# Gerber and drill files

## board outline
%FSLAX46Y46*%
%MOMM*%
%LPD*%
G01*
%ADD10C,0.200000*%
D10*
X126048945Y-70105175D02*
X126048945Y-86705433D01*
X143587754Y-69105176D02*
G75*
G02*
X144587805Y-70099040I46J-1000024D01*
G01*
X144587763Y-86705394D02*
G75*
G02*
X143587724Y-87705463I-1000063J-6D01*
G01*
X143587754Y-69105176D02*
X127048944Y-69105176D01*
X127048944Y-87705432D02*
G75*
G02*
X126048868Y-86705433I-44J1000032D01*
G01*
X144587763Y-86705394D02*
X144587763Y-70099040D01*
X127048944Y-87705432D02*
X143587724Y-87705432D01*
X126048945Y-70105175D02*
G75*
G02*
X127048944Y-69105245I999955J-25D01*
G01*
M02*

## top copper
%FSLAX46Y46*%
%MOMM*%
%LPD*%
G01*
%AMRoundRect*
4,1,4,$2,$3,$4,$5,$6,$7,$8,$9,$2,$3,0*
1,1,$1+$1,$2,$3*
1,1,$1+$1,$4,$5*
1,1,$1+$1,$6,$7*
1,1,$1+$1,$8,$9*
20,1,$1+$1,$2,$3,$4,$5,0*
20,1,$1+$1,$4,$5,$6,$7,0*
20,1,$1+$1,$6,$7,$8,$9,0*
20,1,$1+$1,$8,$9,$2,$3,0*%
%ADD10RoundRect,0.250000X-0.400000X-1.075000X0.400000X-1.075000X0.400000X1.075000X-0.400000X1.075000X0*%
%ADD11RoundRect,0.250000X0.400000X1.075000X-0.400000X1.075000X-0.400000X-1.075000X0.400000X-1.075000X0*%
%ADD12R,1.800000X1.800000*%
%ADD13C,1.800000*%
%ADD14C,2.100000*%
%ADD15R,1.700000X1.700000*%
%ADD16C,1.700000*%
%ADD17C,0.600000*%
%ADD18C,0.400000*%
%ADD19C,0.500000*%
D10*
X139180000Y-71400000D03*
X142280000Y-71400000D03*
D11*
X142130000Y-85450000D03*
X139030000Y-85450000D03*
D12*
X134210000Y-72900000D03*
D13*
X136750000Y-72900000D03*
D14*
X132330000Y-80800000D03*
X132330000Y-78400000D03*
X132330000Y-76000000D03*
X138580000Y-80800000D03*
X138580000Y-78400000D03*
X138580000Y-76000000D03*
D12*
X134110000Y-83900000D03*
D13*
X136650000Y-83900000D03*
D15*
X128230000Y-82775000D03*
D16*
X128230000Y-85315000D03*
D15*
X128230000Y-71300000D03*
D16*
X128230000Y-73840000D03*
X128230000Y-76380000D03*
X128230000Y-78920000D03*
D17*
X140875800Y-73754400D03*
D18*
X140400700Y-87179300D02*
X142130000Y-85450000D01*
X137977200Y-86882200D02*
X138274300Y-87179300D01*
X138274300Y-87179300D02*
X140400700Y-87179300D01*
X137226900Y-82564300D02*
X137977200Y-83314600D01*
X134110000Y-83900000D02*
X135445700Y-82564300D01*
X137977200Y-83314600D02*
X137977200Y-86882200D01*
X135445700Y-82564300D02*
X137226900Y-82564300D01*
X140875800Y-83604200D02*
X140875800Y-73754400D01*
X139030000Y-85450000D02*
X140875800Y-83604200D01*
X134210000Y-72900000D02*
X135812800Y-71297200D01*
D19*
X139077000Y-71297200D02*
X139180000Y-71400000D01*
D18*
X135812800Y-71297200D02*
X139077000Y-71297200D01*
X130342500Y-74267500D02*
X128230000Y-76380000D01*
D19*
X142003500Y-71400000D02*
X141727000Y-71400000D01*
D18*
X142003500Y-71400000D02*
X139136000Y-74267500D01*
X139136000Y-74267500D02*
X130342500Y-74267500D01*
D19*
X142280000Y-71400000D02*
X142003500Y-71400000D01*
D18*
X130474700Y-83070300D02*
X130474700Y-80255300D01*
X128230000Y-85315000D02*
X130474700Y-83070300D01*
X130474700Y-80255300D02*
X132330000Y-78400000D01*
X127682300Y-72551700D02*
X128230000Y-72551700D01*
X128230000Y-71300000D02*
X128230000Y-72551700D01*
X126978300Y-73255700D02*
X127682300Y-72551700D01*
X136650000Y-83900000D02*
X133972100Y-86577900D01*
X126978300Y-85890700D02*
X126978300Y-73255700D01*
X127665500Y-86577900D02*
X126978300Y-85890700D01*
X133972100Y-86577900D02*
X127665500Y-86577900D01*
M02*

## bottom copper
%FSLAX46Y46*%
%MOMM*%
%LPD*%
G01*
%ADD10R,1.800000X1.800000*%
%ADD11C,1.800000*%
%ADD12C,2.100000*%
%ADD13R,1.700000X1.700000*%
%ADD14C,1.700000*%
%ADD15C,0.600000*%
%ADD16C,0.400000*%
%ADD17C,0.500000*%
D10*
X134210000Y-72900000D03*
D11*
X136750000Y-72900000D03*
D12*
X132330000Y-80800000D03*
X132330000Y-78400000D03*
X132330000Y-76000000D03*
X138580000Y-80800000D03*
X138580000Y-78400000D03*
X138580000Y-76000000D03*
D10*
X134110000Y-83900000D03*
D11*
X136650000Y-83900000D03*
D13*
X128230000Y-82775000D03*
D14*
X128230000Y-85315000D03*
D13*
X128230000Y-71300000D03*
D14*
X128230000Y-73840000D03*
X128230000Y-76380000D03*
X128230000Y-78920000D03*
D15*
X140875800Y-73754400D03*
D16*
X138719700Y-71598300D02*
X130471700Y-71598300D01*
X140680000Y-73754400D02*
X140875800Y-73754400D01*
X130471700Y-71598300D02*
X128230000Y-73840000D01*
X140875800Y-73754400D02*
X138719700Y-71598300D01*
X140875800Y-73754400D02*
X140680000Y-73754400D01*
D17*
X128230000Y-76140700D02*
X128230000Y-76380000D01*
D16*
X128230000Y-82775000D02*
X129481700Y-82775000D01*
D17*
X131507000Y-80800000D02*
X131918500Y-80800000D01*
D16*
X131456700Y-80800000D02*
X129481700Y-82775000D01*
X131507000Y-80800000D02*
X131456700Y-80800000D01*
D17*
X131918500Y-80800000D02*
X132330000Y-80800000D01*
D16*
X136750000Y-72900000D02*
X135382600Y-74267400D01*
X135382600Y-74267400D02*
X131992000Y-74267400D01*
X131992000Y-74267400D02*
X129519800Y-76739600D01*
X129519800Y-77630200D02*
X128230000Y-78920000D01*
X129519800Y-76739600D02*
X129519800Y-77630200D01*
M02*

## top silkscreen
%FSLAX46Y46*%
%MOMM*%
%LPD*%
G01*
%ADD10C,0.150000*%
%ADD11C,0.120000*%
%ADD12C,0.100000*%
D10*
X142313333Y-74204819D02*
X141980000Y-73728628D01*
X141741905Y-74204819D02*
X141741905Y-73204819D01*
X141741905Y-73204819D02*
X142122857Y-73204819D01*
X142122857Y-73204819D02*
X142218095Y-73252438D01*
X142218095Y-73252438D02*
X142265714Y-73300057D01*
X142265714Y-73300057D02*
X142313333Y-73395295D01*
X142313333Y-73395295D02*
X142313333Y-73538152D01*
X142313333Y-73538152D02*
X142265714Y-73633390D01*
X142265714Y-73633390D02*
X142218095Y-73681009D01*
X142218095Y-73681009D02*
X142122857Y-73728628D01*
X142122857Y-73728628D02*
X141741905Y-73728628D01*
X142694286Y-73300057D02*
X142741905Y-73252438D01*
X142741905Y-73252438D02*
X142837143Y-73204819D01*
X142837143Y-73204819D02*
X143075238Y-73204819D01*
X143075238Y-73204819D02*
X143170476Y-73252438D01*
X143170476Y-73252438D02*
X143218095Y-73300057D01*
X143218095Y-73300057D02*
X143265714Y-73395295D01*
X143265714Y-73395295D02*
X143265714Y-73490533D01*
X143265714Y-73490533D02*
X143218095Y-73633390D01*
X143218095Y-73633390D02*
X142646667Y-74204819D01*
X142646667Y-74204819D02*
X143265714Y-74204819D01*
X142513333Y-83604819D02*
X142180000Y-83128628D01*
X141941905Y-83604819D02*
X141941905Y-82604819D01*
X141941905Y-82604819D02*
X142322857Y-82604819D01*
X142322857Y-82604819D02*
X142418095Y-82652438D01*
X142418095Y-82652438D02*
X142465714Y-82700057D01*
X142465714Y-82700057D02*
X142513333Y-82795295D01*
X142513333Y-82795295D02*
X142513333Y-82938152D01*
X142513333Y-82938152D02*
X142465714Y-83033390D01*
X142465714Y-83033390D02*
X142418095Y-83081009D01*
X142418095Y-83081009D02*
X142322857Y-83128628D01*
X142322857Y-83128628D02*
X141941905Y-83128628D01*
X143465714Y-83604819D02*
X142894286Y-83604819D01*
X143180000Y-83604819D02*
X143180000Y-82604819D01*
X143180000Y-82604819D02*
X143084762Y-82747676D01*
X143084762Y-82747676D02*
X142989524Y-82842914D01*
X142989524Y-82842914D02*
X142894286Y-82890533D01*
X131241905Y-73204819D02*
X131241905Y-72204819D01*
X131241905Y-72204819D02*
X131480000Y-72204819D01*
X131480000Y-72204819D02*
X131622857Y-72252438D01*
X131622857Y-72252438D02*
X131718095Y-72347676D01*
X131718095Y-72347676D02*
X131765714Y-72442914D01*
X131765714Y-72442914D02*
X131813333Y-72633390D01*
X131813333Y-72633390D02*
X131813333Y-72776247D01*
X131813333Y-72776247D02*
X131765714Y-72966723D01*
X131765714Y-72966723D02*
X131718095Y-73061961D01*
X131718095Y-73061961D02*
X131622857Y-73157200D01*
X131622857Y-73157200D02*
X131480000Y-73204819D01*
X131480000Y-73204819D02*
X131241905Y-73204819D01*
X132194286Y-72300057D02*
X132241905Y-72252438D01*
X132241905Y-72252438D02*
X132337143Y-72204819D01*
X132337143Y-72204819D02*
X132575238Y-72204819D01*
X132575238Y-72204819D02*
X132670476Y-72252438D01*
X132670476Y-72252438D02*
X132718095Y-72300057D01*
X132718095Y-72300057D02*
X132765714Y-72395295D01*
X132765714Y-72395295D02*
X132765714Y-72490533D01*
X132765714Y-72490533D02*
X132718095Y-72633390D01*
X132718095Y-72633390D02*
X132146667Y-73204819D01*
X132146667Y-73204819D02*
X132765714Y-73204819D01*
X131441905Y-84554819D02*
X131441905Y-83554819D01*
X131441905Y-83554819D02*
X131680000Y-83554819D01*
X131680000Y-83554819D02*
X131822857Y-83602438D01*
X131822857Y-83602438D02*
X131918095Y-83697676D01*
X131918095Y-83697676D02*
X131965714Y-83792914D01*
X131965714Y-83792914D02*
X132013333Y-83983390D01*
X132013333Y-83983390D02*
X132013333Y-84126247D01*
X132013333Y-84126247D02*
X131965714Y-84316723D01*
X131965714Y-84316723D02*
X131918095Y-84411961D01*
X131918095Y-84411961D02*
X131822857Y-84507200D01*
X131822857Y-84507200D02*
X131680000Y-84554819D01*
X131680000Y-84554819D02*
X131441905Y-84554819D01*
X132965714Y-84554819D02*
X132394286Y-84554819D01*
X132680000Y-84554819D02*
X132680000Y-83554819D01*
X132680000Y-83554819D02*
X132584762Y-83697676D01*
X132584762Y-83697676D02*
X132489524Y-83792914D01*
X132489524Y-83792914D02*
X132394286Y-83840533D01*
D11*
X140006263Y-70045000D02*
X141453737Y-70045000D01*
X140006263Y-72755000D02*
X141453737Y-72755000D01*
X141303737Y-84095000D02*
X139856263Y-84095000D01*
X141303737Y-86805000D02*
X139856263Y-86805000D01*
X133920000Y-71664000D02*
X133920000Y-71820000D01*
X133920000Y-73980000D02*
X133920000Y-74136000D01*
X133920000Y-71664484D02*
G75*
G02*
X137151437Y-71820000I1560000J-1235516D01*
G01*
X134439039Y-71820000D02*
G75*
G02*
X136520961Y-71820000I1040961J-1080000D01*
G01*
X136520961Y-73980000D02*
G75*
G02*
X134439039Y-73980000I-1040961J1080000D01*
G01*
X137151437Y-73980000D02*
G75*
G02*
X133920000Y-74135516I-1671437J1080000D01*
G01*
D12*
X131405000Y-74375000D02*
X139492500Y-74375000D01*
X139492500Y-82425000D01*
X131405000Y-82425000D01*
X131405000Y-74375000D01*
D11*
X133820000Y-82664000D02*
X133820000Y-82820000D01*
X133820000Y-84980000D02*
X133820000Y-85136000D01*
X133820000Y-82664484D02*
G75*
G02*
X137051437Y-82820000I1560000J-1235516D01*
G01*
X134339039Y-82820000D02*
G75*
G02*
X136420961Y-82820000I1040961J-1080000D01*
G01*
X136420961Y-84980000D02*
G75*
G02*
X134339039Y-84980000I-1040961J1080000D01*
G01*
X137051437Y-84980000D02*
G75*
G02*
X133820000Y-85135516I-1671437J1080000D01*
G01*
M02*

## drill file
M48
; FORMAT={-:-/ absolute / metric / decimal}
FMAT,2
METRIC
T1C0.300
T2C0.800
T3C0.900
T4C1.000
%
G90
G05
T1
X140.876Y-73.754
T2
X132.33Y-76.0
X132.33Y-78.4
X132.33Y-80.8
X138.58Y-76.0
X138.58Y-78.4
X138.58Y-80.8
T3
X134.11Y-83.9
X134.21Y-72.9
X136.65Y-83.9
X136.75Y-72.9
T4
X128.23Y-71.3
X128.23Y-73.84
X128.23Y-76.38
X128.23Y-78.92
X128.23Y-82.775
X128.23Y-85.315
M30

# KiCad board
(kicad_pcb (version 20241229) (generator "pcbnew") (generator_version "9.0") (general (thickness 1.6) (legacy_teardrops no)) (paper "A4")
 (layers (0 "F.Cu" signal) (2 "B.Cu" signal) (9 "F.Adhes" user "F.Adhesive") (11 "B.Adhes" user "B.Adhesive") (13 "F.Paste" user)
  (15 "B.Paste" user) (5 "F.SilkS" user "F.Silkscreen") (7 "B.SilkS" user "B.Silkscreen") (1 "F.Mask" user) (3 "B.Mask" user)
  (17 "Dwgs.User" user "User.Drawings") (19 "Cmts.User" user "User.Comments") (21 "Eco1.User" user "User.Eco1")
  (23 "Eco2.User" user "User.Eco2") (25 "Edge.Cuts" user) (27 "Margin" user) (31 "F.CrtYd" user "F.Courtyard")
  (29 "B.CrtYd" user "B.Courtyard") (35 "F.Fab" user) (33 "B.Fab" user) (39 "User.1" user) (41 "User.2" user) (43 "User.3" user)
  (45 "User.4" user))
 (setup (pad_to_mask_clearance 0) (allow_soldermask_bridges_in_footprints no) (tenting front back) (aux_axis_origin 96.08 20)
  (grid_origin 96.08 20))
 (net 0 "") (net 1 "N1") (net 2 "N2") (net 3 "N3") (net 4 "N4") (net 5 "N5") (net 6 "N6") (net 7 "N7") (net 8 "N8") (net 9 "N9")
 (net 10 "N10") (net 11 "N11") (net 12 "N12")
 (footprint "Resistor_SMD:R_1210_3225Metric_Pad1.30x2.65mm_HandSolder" (layer "F.Cu") (at 140.73 71.4)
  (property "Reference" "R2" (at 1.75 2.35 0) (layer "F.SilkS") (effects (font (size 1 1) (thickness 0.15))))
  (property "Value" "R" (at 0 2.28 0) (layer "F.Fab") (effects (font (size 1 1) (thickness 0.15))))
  (fp_line (start -0.723737 -1.355) (end 0.723737 -1.355) (stroke (width 0.12) (type solid)) (layer "F.SilkS"))
  (fp_line (start -0.723737 1.355) (end 0.723737 1.355) (stroke (width 0.12) (type solid)) (layer "F.SilkS"))
  (pad "1" smd roundrect (at -1.55 0) (size 1.3 2.65) (layers "F.Cu" "F.Mask" "F.Paste") (roundrect_rratio 0.192308) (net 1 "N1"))
  (pad "2" smd roundrect (at 1.55 0) (size 1.3 2.65) (layers "F.Cu" "F.Mask" "F.Paste") (roundrect_rratio 0.192308) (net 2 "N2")))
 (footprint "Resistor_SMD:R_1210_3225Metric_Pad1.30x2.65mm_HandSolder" (layer "F.Cu") (at 140.58 85.45 180)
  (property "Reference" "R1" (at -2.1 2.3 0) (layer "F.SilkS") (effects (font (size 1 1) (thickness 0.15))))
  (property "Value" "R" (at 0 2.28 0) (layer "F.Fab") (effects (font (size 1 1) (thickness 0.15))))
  (fp_line (start -0.723737 1.355) (end 0.723737 1.355) (stroke (width 0.12) (type solid)) (layer "F.SilkS"))
  (fp_line (start -0.723737 -1.355) (end 0.723737 -1.355) (stroke (width 0.12) (type solid)) (layer "F.SilkS"))
  (pad "1" smd roundrect (at -1.55 0 180) (size 1.3 2.65) (layers "F.Cu" "F.Mask" "F.Paste") (roundrect_rratio 0.192308) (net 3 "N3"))
  (pad "2" smd roundrect (at 1.55 0 180) (size 1.3 2.65) (layers "F.Cu" "F.Mask" "F.Paste") (roundrect_rratio 0.192308) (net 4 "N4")))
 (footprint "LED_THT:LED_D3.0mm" (layer "F.Cu") (at 134.21 72.9)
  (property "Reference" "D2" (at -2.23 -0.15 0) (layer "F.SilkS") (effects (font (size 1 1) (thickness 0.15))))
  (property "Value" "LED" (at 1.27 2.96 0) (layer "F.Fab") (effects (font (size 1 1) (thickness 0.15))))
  (fp_line (start -0.29 -1.236) (end -0.29 -1.08) (stroke (width 0.12) (type solid)) (layer "F.SilkS"))
  (fp_line (start -0.29 1.08) (end -0.29 1.236) (stroke (width 0.12) (type solid)) (layer "F.SilkS"))
  (fp_arc (start -0.29 -1.235516) (mid 1.36566 -1.987699) (end 2.941437 -1.08) (stroke (width 0.12) (type solid)) (layer "F.SilkS"))
  (fp_arc (start 0.229039 -1.08) (mid 1.27 -1.5) (end 2.310961 -1.08) (stroke (width 0.12) (type solid)) (layer "F.SilkS"))
  (fp_arc (start 2.310961 1.08) (mid 1.27 1.5) (end 0.229039 1.08) (stroke (width 0.12) (type solid)) (layer "F.SilkS"))
  (fp_arc (start 2.941437 1.08) (mid 1.36566 1.987699) (end -0.29 1.235516) (stroke (width 0.12) (type solid)) (layer "F.SilkS"))
  (pad "1" thru_hole rect (at 0 0) (size 1.8 1.8) (drill 0.9) (layers "*.Cu" "*.Mask") (remove_unused_layers no) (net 1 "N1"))
  (pad "2" thru_hole circle (at 2.54 0) (size 1.8 1.8) (drill 0.9) (layers "*.Cu" "*.Mask") (remove_unused_layers no) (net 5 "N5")))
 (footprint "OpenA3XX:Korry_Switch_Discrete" (layer "F.Cu") (at 141.43 82.5)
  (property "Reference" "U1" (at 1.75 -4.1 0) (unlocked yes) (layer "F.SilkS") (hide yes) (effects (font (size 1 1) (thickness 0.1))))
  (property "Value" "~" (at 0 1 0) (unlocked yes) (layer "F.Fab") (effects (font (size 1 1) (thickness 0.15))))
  (fp_rect (start -10.025 -8.125) (end -1.9375 -0.075) (stroke (width 0.1) (type default)) (fill no) (layer "F.SilkS"))
  (pad "1" thru_hole circle (at -9.1 -1.7) (size 2.1 2.1) (drill 0.8) (layers "*.Cu" "*.Mask") (remove_unused_layers no) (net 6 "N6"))
  (pad "2" thru_hole circle (at -9.1 -4.1) (size 2.1 2.1) (drill 0.8) (layers "*.Cu" "*.Mask") (remove_unused_layers no) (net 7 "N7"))
  (pad "3" thru_hole circle (at -9.1 -6.5) (size 2.1 2.1) (drill 0.8) (layers "*.Cu" "*.Mask") (remove_unused_layers no) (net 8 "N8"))
  (pad "4" thru_hole circle (at -2.85 -1.7) (size 2.1 2.1) (drill 0.8) (layers "*.Cu" "*.Mask") (remove_unused_layers no) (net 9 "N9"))
  (pad "5" thru_hole circle (at -2.85 -4.1) (size 2.1 2.1) (drill 0.8) (layers "*.Cu" "*.Mask") (remove_unused_layers no) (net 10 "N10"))
  (pad "6" thru_hole circle (at -2.85 -6.5) (size 2.1 2.1) (drill 0.8) (layers "*.Cu" "*.Mask") (remove_unused_layers no) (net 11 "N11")))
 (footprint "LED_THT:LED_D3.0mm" (layer "F.Cu") (at 134.11 83.9)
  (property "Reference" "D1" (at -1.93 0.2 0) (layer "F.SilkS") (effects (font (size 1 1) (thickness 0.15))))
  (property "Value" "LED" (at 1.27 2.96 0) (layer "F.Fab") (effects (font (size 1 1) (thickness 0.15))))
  (fp_line (start -0.29 -1.236) (end -0.29 -1.08) (stroke (width 0.12) (type solid)) (layer "F.SilkS"))
  (fp_line (start -0.29 1.08) (end -0.29 1.236) (stroke (width 0.12) (type solid)) (layer "F.SilkS"))
  (fp_arc (start -0.29 -1.235516) (mid 1.36566 -1.987699) (end 2.941437 -1.08) (stroke (width 0.12) (type solid)) (layer "F.SilkS"))
  (fp_arc (start 0.229039 -1.08) (mid 1.27 -1.5) (end 2.310961 -1.08) (stroke (width 0.12) (type solid)) (layer "F.SilkS"))
  (fp_arc (start 2.310961 1.08) (mid 1.27 1.5) (end 0.229039 1.08) (stroke (width 0.12) (type solid)) (layer "F.SilkS"))
  (fp_arc (start 2.941437 1.08) (mid 1.36566 1.987699) (end -0.29 1.235516) (stroke (width 0.12) (type solid)) (layer "F.SilkS"))
  (pad "1" thru_hole rect (at 0 0) (size 1.8 1.8) (drill 0.9) (layers "*.Cu" "*.Mask") (remove_unused_layers no) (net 3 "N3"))
  (pad "2" thru_hole circle (at 2.54 0) (size 1.8 1.8) (drill 0.9) (layers "*.Cu" "*.Mask") (remove_unused_layers no) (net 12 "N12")))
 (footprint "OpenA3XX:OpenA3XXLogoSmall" (layer "B.Cu") (at 135.63 78.2 180)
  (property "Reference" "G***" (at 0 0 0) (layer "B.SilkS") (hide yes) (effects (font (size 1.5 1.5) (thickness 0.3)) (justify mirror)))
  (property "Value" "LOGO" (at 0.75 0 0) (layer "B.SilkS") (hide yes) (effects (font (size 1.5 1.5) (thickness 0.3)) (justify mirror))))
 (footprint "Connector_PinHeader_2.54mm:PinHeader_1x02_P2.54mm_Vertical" (layer "B.Cu") (at 128.23 82.775 180)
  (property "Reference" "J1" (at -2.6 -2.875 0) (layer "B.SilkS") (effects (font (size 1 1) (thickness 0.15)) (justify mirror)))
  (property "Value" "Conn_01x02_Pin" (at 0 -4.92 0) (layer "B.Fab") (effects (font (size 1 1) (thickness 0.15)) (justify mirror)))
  (pad "1" thru_hole rect (at 0 0 180) (size 1.7 1.7) (drill 1) (layers "*.Cu" "*.Mask") (remove_unused_layers no) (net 6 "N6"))
  (pad "2" thru_hole circle (at 0 -2.54 180) (size 1.7 1.7) (drill 1) (layers "*.Cu" "*.Mask") (remove_unused_layers no) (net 7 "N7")))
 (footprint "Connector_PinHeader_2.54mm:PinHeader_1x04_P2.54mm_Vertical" (layer "B.Cu") (at 128.23 71.3 180)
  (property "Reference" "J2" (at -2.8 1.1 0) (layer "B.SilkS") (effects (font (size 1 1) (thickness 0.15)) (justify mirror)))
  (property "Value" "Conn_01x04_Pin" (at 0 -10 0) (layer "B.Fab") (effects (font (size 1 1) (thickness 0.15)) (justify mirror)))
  (pad "1" thru_hole rect (at 0 0 180) (size 1.7 1.7) (drill 1) (layers "*.Cu" "*.Mask") (remove_unused_layers no) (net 12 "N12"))
  (pad "2" thru_hole circle (at 0 -2.54 180) (size 1.7 1.7) (drill 1) (layers "*.Cu" "*.Mask") (remove_unused_layers no) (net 4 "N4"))
  (pad "3" thru_hole circle (at 0 -5.08 180) (size 1.7 1.7) (drill 1) (layers "*.Cu" "*.Mask") (remove_unused_layers no) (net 2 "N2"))
  (pad "4" thru_hole circle (at 0 -7.62 180) (size 1.7 1.7) (drill 1) (layers "*.Cu" "*.Mask") (remove_unused_layers no) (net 5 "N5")))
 (gr_line (start 126.048945 70.105175) (end 126.048945 86.705433) (stroke (width 0.2) (type default)) (layer "Edge.Cuts"))
 (gr_arc (start 143.587754 69.105176) (mid 144.29487 69.398069) (end 144.587763 70.09904) (stroke (width 0.2) (type default))
  (layer "Edge.Cuts"))
 (gr_arc (start 144.587763 86.705394) (mid 144.29486 87.412524) (end 143.587724 87.705432) (stroke (width 0.2) (type default))
  (layer "Edge.Cuts"))
 (gr_line (start 143.587754 69.105176) (end 127.048944 69.105176) (stroke (width 0.2) (type default)) (layer "Edge.Cuts"))
 (gr_arc (start 127.048944 87.705432) (mid 126.341838 87.412539) (end 126.048945 86.705433) (stroke (width 0.2) (type default))
  (layer "Edge.Cuts"))
 (gr_line (start 144.587763 86.705394) (end 144.587763 70.09904) (stroke (width 0.2) (type default)) (layer "Edge.Cuts"))
 (gr_line (start 127.048944 87.705432) (end 143.587724 87.705432) (stroke (width 0.2) (type default)) (layer "Edge.Cuts"))
 (gr_arc (start 126.048945 70.105175) (mid 126.341838 69.398069) (end 127.048944 69.105176) (stroke (width 0.2) (type default))
  (layer "Edge.Cuts"))
 (segment (start 140.4007 87.1793) (end 142.13 85.45) (width 0.4) (layer "F.Cu") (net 3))
 (segment (start 137.9772 86.8822) (end 138.2743 87.1793) (width 0.4) (layer "F.Cu") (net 3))
 (segment (start 138.2743 87.1793) (end 140.4007 87.1793) (width 0.4) (layer "F.Cu") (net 3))
 (segment (start 137.2269 82.5643) (end 137.9772 83.3146) (width 0.4) (layer "F.Cu") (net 3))
 (segment (start 134.11 83.9) (end 135.4457 82.5643) (width 0.4) (layer "F.Cu") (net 3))
 (segment (start 137.9772 83.3146) (end 137.9772 86.8822) (width 0.4) (layer "F.Cu") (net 3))
 (segment (start 135.4457 82.5643) (end 137.2269 82.5643) (width 0.4) (layer "F.Cu") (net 3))
 (segment (start 140.8758 83.6042) (end 140.8758 73.7544) (width 0.4) (layer "F.Cu") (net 4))
 (segment (start 139.03 85.45) (end 140.8758 83.6042) (width 0.4) (layer "F.Cu") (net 4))
 (via (at 140.8758 73.7544) (size 0.6) (drill 0.3) (layers "F.Cu" "B.Cu") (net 4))
 (segment (start 138.7197 71.5983) (end 130.4717 71.5983) (width 0.4) (layer "B.Cu") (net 4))
 (segment (start 140.68 73.7544) (end 140.8758 73.7544) (width 0.4) (layer "B.Cu") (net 4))
 (segment (start 130.4717 71.5983) (end 128.23 73.84) (width 0.4) (layer "B.Cu") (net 4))
 (segment (start 140.8758 73.7544) (end 138.7197 71.5983) (width 0.4) (layer "B.Cu") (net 4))
 (segment (start 140.8758 73.7544) (end 140.68 73.7544) (width 0.4) (layer "B.Cu") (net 4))
 (segment (start 134.21 72.9) (end 135.8128 71.2972) (width 0.4) (layer "F.Cu") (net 1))
 (segment (start 139.077 71.2972) (end 139.18 71.4) (width 0.5) (layer "F.Cu") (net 1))
 (segment (start 135.8128 71.2972) (end 139.077 71.2972) (width 0.4) (layer "F.Cu") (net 1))
 (segment (start 130.3425 74.2675) (end 128.23 76.38) (width 0.4) (layer "F.Cu") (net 2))
 (segment (start 142.0035 71.4) (end 141.727 71.4) (width 0.5) (layer "F.Cu") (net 2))
 (segment (start 142.0035 71.4) (end 139.136 74.2675) (width 0.4) (layer "F.Cu") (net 2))
 (segment (start 139.136 74.2675) (end 130.3425 74.2675) (width 0.4) (layer "F.Cu") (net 2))
 (segment (start 142.28 71.4) (end 142.0035 71.4) (width 0.5) (layer "F.Cu") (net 2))
 (segment (start 128.23 76.1407) (end 128.23 76.38) (width 0.5) (layer "B.Cu") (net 2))
 (segment (start 130.4747 83.0703) (end 130.4747 80.2553) (width 0.4) (layer "F.Cu") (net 7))
 (segment (start 128.23 85.315) (end 130.4747 83.0703) (width 0.4) (layer "F.Cu") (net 7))
 (segment (start 130.4747 80.2553) (end 132.33 78.4) (width 0.4) (layer "F.Cu") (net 7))
 (segment (start 128.23 82.775) (end 129.4817 82.775) (width 0.4) (layer "B.Cu") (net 6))
 (segment (start 131.507 80.8) (end 131.9185 80.8) (width 0.5) (layer "B.Cu") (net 6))
 (segment (start 131.4567 80.8) (end 129.4817 82.775) (width 0.4) (layer "B.Cu") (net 6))
 (segment (start 131.507 80.8) (end 131.4567 80.8) (width 0.4) (layer "B.Cu") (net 6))
 (segment (start 131.9185 80.8) (end 132.33 80.8) (width 0.5) (layer "B.Cu") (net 6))
 (segment (start 127.6823 72.5517) (end 128.23 72.5517) (width 0.4) (layer "F.Cu") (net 12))
 (segment (start 128.23 71.3) (end 128.23 72.5517) (width 0.4) (layer "F.Cu") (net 12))
 (segment (start 126.9783 73.2557) (end 127.6823 72.5517) (width 0.4) (layer "F.Cu") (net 12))
 (segment (start 136.65 83.9) (end 133.9721 86.5779) (width 0.4) (layer "F.Cu") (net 12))
 (segment (start 126.9783 85.8907) (end 126.9783 73.2557) (width 0.4) (layer "F.Cu") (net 12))
 (segment (start 127.6655 86.5779) (end 126.9783 85.8907) (width 0.4) (layer "F.Cu") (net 12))
 (segment (start 133.9721 86.5779) (end 127.6655 86.5779) (width 0.4) (layer "F.Cu") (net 12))
 (segment (start 136.75 72.9) (end 135.3826 74.2674) (width 0.4) (layer "B.Cu") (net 5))
 (segment (start 135.3826 74.2674) (end 131.992 74.2674) (width 0.4) (layer "B.Cu") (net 5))
 (segment (start 131.992 74.2674) (end 129.5198 76.7396) (width 0.4) (layer "B.Cu") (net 5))
 (segment (start 129.5198 77.6302) (end 128.23 78.92) (width 0.4) (layer "B.Cu") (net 5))
 (segment (start 129.5198 76.7396) (end 129.5198 77.6302) (width 0.4) (layer "B.Cu") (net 5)))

